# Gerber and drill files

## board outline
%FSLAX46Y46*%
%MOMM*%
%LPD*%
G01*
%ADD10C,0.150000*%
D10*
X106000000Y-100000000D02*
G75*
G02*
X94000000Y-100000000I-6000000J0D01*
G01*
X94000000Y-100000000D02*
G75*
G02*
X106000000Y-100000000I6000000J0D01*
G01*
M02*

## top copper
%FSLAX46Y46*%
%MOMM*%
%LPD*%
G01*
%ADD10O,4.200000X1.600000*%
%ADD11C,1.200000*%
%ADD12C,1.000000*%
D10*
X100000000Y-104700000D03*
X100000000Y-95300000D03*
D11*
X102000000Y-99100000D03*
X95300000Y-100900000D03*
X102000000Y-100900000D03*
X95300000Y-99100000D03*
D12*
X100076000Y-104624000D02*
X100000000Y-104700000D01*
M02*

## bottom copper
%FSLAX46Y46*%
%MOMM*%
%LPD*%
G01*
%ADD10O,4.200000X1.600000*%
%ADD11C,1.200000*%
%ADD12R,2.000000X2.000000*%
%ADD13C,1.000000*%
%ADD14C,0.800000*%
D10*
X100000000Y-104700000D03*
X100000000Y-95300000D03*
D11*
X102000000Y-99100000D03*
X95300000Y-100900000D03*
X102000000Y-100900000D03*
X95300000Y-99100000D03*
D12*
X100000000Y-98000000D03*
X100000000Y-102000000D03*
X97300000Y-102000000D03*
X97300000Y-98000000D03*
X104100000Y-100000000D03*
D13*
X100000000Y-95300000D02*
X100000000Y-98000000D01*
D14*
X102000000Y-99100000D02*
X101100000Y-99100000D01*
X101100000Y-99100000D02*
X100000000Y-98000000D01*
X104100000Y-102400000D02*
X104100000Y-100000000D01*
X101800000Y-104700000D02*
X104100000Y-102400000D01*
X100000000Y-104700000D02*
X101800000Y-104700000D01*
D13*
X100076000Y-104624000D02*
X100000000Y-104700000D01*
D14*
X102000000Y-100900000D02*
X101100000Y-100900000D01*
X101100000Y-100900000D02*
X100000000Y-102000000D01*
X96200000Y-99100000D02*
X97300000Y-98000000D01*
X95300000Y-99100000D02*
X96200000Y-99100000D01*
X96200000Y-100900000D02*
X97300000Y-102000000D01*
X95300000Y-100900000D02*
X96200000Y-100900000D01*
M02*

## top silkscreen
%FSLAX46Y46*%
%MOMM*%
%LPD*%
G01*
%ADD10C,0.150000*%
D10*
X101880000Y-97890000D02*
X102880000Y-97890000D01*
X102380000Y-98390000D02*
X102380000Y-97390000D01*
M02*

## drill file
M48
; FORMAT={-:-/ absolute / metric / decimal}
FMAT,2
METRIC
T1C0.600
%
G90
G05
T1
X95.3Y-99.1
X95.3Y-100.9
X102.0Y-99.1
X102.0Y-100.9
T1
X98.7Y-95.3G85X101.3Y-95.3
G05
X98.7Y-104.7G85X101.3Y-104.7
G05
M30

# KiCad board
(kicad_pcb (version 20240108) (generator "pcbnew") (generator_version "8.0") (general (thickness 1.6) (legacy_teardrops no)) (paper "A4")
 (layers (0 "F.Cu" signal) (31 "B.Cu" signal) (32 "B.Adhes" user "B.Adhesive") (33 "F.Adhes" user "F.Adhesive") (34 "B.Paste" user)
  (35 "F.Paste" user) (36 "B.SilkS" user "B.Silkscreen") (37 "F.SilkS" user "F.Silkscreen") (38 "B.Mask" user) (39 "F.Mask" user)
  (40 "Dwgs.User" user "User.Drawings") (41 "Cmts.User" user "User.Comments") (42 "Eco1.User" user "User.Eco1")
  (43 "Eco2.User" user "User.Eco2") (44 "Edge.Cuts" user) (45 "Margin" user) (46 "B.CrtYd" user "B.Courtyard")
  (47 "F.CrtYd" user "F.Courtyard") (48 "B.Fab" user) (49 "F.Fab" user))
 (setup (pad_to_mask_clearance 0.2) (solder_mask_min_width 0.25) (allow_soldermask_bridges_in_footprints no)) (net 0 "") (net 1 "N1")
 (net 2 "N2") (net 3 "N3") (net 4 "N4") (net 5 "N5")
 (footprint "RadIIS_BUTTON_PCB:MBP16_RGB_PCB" (layer "F.Cu") (at 100 100)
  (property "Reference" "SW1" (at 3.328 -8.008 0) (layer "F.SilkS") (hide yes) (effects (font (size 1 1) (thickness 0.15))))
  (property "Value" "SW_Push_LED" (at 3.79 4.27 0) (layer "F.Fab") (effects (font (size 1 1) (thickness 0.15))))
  (fp_line (start 1.88 -2.11) (end 2.88 -2.11) (stroke (width 0.15) (type solid)) (layer "F.SilkS"))
  (fp_line (start 2.38 -1.61) (end 2.38 -2.61) (stroke (width 0.15) (type solid)) (layer "F.SilkS"))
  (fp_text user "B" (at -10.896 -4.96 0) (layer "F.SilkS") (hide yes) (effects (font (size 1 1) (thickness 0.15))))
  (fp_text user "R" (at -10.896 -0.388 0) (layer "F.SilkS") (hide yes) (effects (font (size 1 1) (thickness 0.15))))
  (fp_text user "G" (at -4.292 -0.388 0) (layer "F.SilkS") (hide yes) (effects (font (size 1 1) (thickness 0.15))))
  (pad "1" thru_hole oval (at 0 4.7) (size 4.2 1.6) (drill oval 3.2 0.6) (layers "*.Cu" "*.Mask") (remove_unused_layers no) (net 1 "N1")
   (solder_mask_margin 0.05))
  (pad "2" thru_hole oval (at 0 -4.7) (size 4.2 1.6) (drill oval 3.2 0.6) (layers "*.Cu" "*.Mask") (remove_unused_layers no) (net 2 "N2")
   (solder_mask_margin 0.05))
  (pad "3" thru_hole circle (at 2 -0.9) (size 1.2 1.2) (drill 0.6) (layers "*.Cu" "*.Mask") (remove_unused_layers no) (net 2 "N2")
   (solder_mask_margin 0.05))
  (pad "4" thru_hole circle (at -4.7 0.9) (size 1.2 1.2) (drill 0.6) (layers "*.Cu" "*.Mask") (remove_unused_layers no) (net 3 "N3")
   (solder_mask_margin 0.05))
  (pad "5" thru_hole circle (at 2 0.9) (size 1.2 1.2) (drill 0.6) (layers "*.Cu" "*.Mask") (remove_unused_layers no) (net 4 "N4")
   (solder_mask_margin 0.05))
  (pad "6" thru_hole circle (at -4.7 -0.9) (size 1.2 1.2) (drill 0.6) (layers "*.Cu" "*.Mask") (remove_unused_layers no) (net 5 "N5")
   (solder_mask_margin 0.05)))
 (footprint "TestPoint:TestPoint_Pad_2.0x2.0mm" (layer "B.Cu") (at 100 98)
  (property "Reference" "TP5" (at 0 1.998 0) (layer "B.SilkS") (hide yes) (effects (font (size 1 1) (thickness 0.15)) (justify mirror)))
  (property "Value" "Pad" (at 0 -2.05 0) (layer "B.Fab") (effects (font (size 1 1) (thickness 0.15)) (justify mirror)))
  (pad "1" smd rect (at 0 0) (size 2 2) (layers "B.Cu" "B.Mask") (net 2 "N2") (solder_mask_margin 0.05)))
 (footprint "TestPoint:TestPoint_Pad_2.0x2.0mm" (layer "B.Cu") (at 100 102 -90)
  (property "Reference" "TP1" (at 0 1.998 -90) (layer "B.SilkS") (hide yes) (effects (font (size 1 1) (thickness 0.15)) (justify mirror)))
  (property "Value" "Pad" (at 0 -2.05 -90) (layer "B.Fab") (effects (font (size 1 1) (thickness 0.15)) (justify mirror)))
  (pad "1" smd rect (at 0 0 270) (size 2 2) (layers "B.Cu" "B.Mask") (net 4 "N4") (solder_mask_margin 0.05)))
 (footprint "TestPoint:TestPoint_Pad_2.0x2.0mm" (layer "B.Cu") (at 97.3 102)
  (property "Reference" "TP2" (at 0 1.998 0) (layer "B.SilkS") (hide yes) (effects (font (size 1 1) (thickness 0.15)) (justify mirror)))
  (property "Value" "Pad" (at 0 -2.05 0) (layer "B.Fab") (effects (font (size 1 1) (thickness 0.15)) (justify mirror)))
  (pad "1" smd rect (at 0 0) (size 2 2) (layers "B.Cu" "B.Mask") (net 3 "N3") (solder_mask_margin 0.05)))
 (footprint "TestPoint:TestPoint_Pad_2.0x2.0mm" (layer "B.Cu") (at 97.3 98)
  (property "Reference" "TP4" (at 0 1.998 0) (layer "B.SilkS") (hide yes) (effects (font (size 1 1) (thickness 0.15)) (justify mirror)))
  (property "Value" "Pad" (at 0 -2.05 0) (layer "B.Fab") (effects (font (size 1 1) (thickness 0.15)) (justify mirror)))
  (pad "1" smd rect (at 0 0) (size 2 2) (layers "B.Cu" "B.Mask") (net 5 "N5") (solder_mask_margin 0.05)))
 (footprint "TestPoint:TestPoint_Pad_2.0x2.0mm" (layer "B.Cu") (at 104.1 100)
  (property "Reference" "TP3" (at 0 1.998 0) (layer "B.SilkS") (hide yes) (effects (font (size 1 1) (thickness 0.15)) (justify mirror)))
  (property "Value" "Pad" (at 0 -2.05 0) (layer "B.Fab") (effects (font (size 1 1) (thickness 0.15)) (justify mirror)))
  (pad "1" smd rect (at 0 0) (size 2 2) (layers "B.Cu" "B.Mask") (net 1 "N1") (solder_mask_margin 0.05)))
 (gr_circle (center 100 100) (end 106 100) (stroke (width 0.15) (type solid)) (fill none) (layer "Edge.Cuts"))
 (segment (start 100 95.3) (end 100 98) (width 1) (layer "B.Cu") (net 2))
 (segment (start 102 99.1) (end 101.1 99.1) (width 0.8) (layer "B.Cu") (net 2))
 (segment (start 101.1 99.1) (end 100 98) (width 0.8) (layer "B.Cu") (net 2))
 (segment (start 100.076 104.624) (end 100 104.7) (width 1) (layer "F.Cu") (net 1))
 (segment (start 104.1 102.4) (end 104.1 100) (width 0.8) (layer "B.Cu") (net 1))
 (segment (start 101.8 104.7) (end 104.1 102.4) (width 0.8) (layer "B.Cu") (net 1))
 (segment (start 100 104.7) (end 101.8 104.7) (width 0.8) (layer "B.Cu") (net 1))
 (segment (start 100.076 104.624) (end 100 104.7) (width 1) (layer "B.Cu") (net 1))
 (segment (start 102 100.9) (end 101.1 100.9) (width 0.8) (layer "B.Cu") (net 4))
 (segment (start 101.1 100.9) (end 100 102) (width 0.8) (layer "B.Cu") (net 4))
 (segment (start 96.2 99.1) (end 97.3 98) (width 0.8) (layer "B.Cu") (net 5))
 (segment (start 95.3 99.1) (end 96.2 99.1) (width 0.8) (layer "B.Cu") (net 5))
 (segment (start 96.2 100.9) (end 97.3 102) (width 0.8) (layer "B.Cu") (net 3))
 (segment (start 95.3 100.9) (end 96.2 100.9) (width 0.8) (layer "B.Cu") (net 3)))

